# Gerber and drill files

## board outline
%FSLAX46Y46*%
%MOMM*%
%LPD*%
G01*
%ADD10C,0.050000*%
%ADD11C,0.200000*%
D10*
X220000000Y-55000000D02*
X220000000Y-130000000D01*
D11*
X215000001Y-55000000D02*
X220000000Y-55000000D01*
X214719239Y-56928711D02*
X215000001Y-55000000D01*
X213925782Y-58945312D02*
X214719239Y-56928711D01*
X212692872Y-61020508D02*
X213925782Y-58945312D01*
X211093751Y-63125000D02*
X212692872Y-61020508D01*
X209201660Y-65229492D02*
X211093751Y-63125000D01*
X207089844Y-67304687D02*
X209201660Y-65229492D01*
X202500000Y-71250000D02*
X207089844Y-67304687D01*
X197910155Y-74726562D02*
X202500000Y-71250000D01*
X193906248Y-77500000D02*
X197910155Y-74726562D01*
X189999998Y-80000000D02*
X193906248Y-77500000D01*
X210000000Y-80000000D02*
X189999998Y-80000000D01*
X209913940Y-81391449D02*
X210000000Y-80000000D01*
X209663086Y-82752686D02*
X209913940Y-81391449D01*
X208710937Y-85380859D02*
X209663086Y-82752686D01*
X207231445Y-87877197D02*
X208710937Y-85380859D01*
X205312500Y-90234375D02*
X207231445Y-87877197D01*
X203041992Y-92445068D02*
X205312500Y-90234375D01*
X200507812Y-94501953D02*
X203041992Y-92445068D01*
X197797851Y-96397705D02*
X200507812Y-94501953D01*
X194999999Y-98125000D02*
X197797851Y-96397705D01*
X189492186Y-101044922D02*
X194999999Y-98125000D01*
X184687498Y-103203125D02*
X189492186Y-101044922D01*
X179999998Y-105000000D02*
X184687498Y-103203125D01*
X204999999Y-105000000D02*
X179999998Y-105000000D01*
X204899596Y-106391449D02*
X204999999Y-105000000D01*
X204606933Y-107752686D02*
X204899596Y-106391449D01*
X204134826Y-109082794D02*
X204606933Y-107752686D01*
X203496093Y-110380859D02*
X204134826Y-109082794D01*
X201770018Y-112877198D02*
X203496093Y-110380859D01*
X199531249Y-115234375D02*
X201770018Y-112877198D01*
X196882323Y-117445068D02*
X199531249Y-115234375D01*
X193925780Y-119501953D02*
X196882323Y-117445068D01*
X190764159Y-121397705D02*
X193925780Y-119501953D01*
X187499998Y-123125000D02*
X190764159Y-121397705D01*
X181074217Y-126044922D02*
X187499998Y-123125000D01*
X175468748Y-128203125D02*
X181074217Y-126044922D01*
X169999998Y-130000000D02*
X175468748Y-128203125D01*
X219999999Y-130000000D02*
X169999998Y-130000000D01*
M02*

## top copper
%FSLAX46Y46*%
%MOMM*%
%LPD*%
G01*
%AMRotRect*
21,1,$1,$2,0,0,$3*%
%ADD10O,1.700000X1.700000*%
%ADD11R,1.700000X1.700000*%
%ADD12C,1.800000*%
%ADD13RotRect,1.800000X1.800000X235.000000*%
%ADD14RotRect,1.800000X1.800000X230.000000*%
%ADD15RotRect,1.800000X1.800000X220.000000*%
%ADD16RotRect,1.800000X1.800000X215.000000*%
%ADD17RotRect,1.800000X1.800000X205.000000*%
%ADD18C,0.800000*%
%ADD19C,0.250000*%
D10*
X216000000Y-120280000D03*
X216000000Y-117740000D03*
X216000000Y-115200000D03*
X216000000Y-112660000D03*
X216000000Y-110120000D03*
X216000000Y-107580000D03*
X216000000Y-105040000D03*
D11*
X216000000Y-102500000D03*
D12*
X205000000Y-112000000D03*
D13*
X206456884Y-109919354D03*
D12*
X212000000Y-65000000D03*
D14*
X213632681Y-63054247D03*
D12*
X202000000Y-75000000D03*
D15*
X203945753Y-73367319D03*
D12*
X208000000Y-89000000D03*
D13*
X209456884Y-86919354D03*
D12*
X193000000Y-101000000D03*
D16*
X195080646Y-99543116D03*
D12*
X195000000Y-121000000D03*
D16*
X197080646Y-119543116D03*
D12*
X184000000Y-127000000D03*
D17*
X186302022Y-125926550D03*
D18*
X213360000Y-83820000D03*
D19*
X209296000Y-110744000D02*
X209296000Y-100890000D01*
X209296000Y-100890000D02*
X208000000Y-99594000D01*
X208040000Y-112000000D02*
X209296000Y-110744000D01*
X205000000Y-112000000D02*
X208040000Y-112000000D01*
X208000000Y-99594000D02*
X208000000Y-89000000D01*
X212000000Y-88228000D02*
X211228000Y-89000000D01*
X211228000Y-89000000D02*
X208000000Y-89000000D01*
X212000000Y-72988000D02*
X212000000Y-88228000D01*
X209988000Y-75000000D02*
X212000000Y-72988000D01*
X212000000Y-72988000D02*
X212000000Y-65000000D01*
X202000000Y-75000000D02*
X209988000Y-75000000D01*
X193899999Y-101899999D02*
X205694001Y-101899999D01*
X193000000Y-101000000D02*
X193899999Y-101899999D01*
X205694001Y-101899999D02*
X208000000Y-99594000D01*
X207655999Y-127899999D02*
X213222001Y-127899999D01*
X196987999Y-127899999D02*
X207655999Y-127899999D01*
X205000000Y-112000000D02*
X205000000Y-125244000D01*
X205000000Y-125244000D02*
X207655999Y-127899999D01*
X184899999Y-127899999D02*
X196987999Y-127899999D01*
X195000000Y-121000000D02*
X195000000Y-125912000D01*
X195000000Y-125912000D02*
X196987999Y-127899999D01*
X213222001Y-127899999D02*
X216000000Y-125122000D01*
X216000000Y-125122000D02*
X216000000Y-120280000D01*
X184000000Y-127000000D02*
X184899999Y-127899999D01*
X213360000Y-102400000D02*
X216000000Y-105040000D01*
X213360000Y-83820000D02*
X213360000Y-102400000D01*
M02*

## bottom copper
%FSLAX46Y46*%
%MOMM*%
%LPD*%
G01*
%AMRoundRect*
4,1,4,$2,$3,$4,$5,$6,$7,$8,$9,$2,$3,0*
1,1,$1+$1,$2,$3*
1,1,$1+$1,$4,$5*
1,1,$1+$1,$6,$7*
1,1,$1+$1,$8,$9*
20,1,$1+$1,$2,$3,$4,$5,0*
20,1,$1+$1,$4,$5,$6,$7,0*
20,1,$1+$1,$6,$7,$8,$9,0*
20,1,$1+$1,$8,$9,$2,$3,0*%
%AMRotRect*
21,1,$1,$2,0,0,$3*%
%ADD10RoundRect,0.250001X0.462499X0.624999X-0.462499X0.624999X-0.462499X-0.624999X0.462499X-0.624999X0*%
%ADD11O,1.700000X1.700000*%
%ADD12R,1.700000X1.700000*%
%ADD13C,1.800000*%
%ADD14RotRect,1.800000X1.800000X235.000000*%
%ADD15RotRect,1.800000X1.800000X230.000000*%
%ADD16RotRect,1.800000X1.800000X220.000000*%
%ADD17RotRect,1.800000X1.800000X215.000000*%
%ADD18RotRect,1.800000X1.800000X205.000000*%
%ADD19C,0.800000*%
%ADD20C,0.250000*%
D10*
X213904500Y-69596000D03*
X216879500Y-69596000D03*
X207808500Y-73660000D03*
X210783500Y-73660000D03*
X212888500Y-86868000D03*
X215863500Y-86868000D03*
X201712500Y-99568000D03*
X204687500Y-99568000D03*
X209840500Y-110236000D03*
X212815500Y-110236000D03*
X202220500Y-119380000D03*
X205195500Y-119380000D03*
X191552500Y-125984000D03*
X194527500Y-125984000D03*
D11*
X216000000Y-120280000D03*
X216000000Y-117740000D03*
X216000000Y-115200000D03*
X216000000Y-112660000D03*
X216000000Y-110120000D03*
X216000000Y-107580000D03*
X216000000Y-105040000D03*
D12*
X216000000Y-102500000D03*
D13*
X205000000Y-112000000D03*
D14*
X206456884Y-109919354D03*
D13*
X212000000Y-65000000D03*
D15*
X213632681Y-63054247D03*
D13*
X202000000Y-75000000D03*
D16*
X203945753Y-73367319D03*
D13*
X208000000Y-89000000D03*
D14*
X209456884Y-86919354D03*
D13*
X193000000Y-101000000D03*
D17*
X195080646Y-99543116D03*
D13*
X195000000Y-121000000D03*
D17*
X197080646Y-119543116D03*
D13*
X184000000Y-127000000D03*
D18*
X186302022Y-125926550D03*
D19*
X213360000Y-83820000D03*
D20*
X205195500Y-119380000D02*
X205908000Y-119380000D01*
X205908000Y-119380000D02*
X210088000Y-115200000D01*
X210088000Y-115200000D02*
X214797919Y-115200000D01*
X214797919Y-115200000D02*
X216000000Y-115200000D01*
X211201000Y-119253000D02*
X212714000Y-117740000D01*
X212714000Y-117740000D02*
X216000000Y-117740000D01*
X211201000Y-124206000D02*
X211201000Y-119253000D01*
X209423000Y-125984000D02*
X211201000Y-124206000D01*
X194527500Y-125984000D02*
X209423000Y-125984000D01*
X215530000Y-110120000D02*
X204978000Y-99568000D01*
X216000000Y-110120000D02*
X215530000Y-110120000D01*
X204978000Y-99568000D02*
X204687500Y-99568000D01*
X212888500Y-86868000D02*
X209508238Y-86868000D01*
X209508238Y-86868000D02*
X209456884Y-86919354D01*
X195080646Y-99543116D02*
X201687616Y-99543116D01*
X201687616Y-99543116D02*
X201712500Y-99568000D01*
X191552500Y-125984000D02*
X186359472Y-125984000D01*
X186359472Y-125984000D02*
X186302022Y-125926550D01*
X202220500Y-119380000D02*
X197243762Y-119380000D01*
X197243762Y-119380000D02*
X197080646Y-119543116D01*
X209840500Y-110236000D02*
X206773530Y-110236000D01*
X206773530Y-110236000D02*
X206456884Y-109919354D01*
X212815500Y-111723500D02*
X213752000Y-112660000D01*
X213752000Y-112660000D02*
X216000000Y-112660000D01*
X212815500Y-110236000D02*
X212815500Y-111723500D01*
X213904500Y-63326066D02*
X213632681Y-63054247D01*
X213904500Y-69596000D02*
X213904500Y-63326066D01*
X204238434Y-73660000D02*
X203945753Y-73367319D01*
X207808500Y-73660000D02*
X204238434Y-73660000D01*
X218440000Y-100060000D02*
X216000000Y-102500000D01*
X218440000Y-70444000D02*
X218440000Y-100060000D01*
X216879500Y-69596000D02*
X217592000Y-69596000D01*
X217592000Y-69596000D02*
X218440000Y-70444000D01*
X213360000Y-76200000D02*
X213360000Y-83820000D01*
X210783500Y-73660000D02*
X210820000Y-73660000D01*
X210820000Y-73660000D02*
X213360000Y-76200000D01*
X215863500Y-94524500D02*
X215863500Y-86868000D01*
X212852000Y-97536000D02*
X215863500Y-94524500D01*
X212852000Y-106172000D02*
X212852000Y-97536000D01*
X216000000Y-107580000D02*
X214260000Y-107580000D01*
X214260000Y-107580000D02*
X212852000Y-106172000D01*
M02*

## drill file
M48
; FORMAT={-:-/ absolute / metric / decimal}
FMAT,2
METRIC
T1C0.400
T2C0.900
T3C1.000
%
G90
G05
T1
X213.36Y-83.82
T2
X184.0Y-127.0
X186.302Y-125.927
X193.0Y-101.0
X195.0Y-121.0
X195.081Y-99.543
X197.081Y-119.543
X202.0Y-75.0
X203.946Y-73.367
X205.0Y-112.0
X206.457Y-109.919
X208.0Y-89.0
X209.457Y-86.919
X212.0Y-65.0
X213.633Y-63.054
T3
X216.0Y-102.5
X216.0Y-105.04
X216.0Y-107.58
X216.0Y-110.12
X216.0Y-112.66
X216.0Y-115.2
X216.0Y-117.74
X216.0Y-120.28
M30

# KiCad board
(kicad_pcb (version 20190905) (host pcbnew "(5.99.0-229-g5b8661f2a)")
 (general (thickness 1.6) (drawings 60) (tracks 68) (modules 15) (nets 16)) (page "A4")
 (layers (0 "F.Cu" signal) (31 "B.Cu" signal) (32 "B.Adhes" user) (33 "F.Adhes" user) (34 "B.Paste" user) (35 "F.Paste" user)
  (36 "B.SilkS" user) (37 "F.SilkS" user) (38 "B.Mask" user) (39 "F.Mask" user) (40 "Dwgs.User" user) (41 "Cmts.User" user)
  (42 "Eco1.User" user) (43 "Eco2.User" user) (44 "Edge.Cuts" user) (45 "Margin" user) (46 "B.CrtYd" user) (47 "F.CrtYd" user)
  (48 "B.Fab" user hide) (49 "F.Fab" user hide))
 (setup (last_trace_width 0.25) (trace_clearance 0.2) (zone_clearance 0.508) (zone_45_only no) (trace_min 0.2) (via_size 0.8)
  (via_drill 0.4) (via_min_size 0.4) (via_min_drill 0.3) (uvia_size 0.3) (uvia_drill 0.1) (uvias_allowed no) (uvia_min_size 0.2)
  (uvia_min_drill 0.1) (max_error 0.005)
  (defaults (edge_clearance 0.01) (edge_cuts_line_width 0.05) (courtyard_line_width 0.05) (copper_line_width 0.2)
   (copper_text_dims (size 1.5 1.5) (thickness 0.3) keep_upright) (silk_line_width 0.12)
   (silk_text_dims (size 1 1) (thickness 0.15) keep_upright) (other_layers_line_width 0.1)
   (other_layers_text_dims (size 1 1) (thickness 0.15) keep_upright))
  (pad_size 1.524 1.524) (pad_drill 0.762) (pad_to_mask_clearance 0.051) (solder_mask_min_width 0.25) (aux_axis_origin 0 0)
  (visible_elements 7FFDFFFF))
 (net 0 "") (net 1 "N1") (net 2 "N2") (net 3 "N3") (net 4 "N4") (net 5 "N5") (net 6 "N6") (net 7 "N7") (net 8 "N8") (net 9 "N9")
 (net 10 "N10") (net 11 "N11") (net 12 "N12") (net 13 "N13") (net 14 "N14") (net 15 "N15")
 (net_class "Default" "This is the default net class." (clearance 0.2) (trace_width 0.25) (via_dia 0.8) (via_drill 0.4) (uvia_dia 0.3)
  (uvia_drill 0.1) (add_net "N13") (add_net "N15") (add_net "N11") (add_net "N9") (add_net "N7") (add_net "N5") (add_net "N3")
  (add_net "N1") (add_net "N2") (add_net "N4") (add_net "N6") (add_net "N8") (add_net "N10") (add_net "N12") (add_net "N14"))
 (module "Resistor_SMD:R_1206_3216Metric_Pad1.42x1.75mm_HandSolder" (layer "B.Cu") (at 215.392 69.596 180)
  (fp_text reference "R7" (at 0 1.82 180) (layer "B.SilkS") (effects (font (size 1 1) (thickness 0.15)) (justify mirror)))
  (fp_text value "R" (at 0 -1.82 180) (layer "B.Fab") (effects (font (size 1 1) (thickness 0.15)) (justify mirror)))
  (pad "2" smd roundrect (at 1.4875 0 180) (size 1.425 1.75) (layers "B.Cu" "B.Paste" "B.Mask") (roundrect_rratio 0.175439) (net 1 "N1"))
  (pad "1" smd roundrect (at -1.4875 0 180) (size 1.425 1.75) (layers "B.Cu" "B.Paste" "B.Mask") (roundrect_rratio 0.175439) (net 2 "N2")))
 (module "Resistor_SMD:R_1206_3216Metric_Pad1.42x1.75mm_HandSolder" (layer "B.Cu") (at 209.296 73.66 180)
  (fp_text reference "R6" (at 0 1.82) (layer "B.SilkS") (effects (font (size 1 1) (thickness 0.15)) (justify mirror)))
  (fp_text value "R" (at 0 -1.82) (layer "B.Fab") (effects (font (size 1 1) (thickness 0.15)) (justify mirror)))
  (pad "2" smd roundrect (at 1.4875 0 180) (size 1.425 1.75) (layers "B.Cu" "B.Paste" "B.Mask") (roundrect_rratio 0.175439) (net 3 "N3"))
  (pad "1" smd roundrect (at -1.4875 0 180) (size 1.425 1.75) (layers "B.Cu" "B.Paste" "B.Mask") (roundrect_rratio 0.175439) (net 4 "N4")))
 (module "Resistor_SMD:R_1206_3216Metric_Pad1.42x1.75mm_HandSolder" (layer "B.Cu") (at 214.376 86.868 180)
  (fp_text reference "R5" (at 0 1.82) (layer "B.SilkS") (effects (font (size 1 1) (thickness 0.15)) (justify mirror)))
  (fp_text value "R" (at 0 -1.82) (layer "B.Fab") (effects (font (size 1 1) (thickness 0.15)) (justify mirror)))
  (pad "2" smd roundrect (at 1.4875 0 180) (size 1.425 1.75) (layers "B.Cu" "B.Paste" "B.Mask") (roundrect_rratio 0.175439) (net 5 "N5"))
  (pad "1" smd roundrect (at -1.4875 0 180) (size 1.425 1.75) (layers "B.Cu" "B.Paste" "B.Mask") (roundrect_rratio 0.175439) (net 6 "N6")))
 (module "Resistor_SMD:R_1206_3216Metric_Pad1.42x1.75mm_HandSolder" (layer "B.Cu") (at 203.2 99.568 180)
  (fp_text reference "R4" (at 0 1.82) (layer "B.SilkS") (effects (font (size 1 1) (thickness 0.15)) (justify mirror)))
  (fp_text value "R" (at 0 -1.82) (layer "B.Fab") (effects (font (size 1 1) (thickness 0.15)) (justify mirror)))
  (pad "2" smd roundrect (at 1.4875 0 180) (size 1.425 1.75) (layers "B.Cu" "B.Paste" "B.Mask") (roundrect_rratio 0.175439) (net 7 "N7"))
  (pad "1" smd roundrect (at -1.4875 0 180) (size 1.425 1.75) (layers "B.Cu" "B.Paste" "B.Mask") (roundrect_rratio 0.175439) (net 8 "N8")))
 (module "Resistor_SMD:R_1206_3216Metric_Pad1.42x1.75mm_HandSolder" (layer "B.Cu") (at 211.328 110.236 180)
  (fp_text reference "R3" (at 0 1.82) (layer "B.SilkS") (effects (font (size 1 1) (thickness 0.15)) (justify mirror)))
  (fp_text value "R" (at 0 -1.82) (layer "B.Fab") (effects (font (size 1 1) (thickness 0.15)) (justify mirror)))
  (pad "2" smd roundrect (at 1.4875 0 180) (size 1.425 1.75) (layers "B.Cu" "B.Paste" "B.Mask") (roundrect_rratio 0.175439) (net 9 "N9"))
  (pad "1" smd roundrect (at -1.4875 0 180) (size 1.425 1.75) (layers "B.Cu" "B.Paste" "B.Mask") (roundrect_rratio 0.175439) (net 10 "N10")))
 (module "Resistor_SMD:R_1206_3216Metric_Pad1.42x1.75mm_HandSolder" (layer "B.Cu") (at 203.708 119.38 180)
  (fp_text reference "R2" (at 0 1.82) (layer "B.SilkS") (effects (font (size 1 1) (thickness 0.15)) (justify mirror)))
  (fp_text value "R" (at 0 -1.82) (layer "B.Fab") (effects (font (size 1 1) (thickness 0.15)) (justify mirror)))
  (pad "2" smd roundrect (at 1.4875 0 180) (size 1.425 1.75) (layers "B.Cu" "B.Paste" "B.Mask") (roundrect_rratio 0.175439) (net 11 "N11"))
  (pad "1" smd roundrect (at -1.4875 0 180) (size 1.425 1.75) (layers "B.Cu" "B.Paste" "B.Mask") (roundrect_rratio 0.175439) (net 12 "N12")))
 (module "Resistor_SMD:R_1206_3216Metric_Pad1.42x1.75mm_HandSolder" (layer "B.Cu") (at 193.04 125.984 180)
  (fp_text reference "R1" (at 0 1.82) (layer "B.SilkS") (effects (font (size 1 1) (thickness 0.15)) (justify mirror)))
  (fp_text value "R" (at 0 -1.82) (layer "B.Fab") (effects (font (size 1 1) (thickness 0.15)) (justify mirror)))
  (pad "2" smd roundrect (at 1.4875 0 180) (size 1.425 1.75) (layers "B.Cu" "B.Paste" "B.Mask") (roundrect_rratio 0.175439) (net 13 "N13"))
  (pad "1" smd roundrect (at -1.4875 0 180) (size 1.425 1.75) (layers "B.Cu" "B.Paste" "B.Mask") (roundrect_rratio 0.175439) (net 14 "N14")))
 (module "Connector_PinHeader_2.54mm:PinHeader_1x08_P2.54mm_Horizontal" (layer "F.Cu") (at 216 102.5)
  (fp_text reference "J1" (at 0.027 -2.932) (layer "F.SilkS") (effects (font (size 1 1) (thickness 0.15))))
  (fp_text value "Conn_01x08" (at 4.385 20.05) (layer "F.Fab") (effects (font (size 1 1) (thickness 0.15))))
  (pad "8" thru_hole oval (at 0 17.78) (size 1.7 1.7) (drill 1) (layers *.Cu *.Mask) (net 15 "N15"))
  (pad "7" thru_hole oval (at 0 15.24) (size 1.7 1.7) (drill 1) (layers *.Cu *.Mask) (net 14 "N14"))
  (pad "6" thru_hole oval (at 0 12.7) (size 1.7 1.7) (drill 1) (layers *.Cu *.Mask) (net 12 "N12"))
  (pad "5" thru_hole oval (at 0 10.16) (size 1.7 1.7) (drill 1) (layers *.Cu *.Mask) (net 10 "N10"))
  (pad "4" thru_hole oval (at 0 7.62) (size 1.7 1.7) (drill 1) (layers *.Cu *.Mask) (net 8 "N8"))
  (pad "3" thru_hole oval (at 0 5.08) (size 1.7 1.7) (drill 1) (layers *.Cu *.Mask) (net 6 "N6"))
  (pad "2" thru_hole oval (at 0 2.54) (size 1.7 1.7) (drill 1) (layers *.Cu *.Mask) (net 4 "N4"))
  (pad "1" thru_hole rect (at 0 0) (size 1.7 1.7) (drill 1) (layers *.Cu *.Mask) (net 2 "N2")))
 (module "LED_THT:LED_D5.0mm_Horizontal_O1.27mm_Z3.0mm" (layer "F.Cu") (at 206.456884 109.919354 -125)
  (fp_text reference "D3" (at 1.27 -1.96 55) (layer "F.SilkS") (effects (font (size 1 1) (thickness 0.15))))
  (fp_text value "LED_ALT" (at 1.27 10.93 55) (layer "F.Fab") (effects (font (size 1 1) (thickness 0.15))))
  (pad "2" thru_hole circle (at 2.54 0 235) (size 1.8 1.8) (drill 0.9) (layers *.Cu *.Mask) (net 15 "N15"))
  (pad "1" thru_hole rect (at 0 0 235) (size 1.8 1.8) (drill 0.9) (layers *.Cu *.Mask) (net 9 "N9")))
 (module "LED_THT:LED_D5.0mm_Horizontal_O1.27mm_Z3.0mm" (layer "F.Cu") (at 213.632681 63.054247 -130)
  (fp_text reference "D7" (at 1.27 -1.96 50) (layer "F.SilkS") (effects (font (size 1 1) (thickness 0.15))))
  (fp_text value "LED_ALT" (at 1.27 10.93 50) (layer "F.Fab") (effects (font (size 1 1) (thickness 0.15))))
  (pad "2" thru_hole circle (at 2.54 0 230) (size 1.8 1.8) (drill 0.9) (layers *.Cu *.Mask) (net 15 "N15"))
  (pad "1" thru_hole rect (at 0 0 230) (size 1.8 1.8) (drill 0.9) (layers *.Cu *.Mask) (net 1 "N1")))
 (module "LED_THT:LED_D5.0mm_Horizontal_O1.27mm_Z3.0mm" (layer "F.Cu") (at 203.945753 73.367319 -140)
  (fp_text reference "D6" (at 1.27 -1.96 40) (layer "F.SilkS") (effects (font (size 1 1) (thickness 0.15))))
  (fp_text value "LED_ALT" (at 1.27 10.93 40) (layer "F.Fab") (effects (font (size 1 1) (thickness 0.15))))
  (pad "2" thru_hole circle (at 2.54 0 220) (size 1.8 1.8) (drill 0.9) (layers *.Cu *.Mask) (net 15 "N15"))
  (pad "1" thru_hole rect (at 0 0 220) (size 1.8 1.8) (drill 0.9) (layers *.Cu *.Mask) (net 3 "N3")))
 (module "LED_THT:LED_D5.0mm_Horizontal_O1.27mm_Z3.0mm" (layer "F.Cu") (at 209.456884 86.919354 -125)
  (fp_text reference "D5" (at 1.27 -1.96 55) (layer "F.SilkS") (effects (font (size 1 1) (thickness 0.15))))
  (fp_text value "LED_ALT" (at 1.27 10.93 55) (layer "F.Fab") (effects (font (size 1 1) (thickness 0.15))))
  (pad "2" thru_hole circle (at 2.54 0 235) (size 1.8 1.8) (drill 0.9) (layers *.Cu *.Mask) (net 15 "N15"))
  (pad "1" thru_hole rect (at 0 0 235) (size 1.8 1.8) (drill 0.9) (layers *.Cu *.Mask) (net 5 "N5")))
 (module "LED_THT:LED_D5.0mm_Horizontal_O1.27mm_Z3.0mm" (layer "F.Cu") (at 195.080646 99.543116 -145)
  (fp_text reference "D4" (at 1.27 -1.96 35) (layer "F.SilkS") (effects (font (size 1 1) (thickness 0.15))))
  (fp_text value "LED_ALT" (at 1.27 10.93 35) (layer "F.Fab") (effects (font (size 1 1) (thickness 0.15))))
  (pad "2" thru_hole circle (at 2.54 0 215) (size 1.8 1.8) (drill 0.9) (layers *.Cu *.Mask) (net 15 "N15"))
  (pad "1" thru_hole rect (at 0 0 215) (size 1.8 1.8) (drill 0.9) (layers *.Cu *.Mask) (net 7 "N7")))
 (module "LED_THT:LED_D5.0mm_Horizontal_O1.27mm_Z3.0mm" (layer "F.Cu") (at 197.080646 119.543116 -145)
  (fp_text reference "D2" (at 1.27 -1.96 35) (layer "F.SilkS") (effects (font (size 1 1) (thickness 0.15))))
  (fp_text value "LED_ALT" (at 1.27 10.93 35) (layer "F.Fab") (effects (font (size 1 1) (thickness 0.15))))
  (pad "2" thru_hole circle (at 2.54 0 215) (size 1.8 1.8) (drill 0.9) (layers *.Cu *.Mask) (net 15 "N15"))
  (pad "1" thru_hole rect (at 0 0 215) (size 1.8 1.8) (drill 0.9) (layers *.Cu *.Mask) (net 11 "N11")))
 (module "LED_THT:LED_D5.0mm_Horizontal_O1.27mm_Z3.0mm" (layer "F.Cu") (at 186.302022 125.92655 -155)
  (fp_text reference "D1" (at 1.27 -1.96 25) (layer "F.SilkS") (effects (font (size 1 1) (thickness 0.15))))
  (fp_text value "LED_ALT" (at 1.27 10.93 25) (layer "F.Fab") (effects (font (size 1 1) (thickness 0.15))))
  (pad "2" thru_hole circle (at 2.54 0 205) (size 1.8 1.8) (drill 0.9) (layers *.Cu *.Mask) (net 15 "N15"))
  (pad "1" thru_hole rect (at 0 0 205) (size 1.8 1.8) (drill 0.9) (layers *.Cu *.Mask) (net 13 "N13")))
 (gr_line (start 220 55) (end 220 130) (layer "Edge.Cuts") (width 0.05))
 (gr_line (start 215.000001 55) (end 220 55) (layer "Edge.Cuts") (width 0.2))
 (gr_line (start 214.719239 56.928711) (end 215.000001 55) (layer "Edge.Cuts") (width 0.2))
 (gr_line (start 213.925782 58.945312) (end 214.719239 56.928711) (layer "Edge.Cuts") (width 0.2))
 (gr_line (start 212.692872 61.020508) (end 213.925782 58.945312) (layer "Edge.Cuts") (width 0.2))
 (gr_line (start 211.093751 63.125) (end 212.692872 61.020508) (layer "Edge.Cuts") (width 0.2))
 (gr_line (start 209.20166 65.229492) (end 211.093751 63.125) (layer "Edge.Cuts") (width 0.2))
 (gr_line (start 207.089844 67.304687) (end 209.20166 65.229492) (layer "Edge.Cuts") (width 0.2))
 (gr_line (start 202.5 71.25) (end 207.089844 67.304687) (layer "Edge.Cuts") (width 0.2))
 (gr_line (start 197.910155 74.726562) (end 202.5 71.25) (layer "Edge.Cuts") (width 0.2))
 (gr_line (start 193.906248 77.5) (end 197.910155 74.726562) (layer "Edge.Cuts") (width 0.2))
 (gr_line (start 189.999998 80) (end 193.906248 77.5) (layer "Edge.Cuts") (width 0.2))
 (gr_line (start 210 80) (end 189.999998 80) (layer "Edge.Cuts") (width 0.2))
 (gr_line (start 209.91394 81.391449) (end 210 80) (layer "Edge.Cuts") (width 0.2))
 (gr_line (start 209.663086 82.752686) (end 209.91394 81.391449) (layer "Edge.Cuts") (width 0.2))
 (gr_line (start 208.710937 85.380859) (end 209.663086 82.752686) (layer "Edge.Cuts") (width 0.2))
 (gr_line (start 207.231445 87.877197) (end 208.710937 85.380859) (layer "Edge.Cuts") (width 0.2))
 (gr_line (start 205.3125 90.234375) (end 207.231445 87.877197) (layer "Edge.Cuts") (width 0.2))
 (gr_line (start 203.041992 92.445068) (end 205.3125 90.234375) (layer "Edge.Cuts") (width 0.2))
 (gr_line (start 200.507812 94.501953) (end 203.041992 92.445068) (layer "Edge.Cuts") (width 0.2))
 (gr_line (start 197.797851 96.397705) (end 200.507812 94.501953) (layer "Edge.Cuts") (width 0.2))
 (gr_line (start 194.999999 98.125) (end 197.797851 96.397705) (layer "Edge.Cuts") (width 0.2))
 (gr_line (start 189.492186 101.044922) (end 194.999999 98.125) (layer "Edge.Cuts") (width 0.2))
 (gr_line (start 184.687498 103.203125) (end 189.492186 101.044922) (layer "Edge.Cuts") (width 0.2))
 (gr_line (start 179.999998 105) (end 184.687498 103.203125) (layer "Edge.Cuts") (width 0.2))
 (gr_line (start 204.999999 105) (end 179.999998 105) (layer "Edge.Cuts") (width 0.2))
 (gr_line (start 204.899596 106.391449) (end 204.999999 105) (layer "Edge.Cuts") (width 0.2))
 (gr_line (start 204.606933 107.752686) (end 204.899596 106.391449) (layer "Edge.Cuts") (width 0.2))
 (gr_line (start 204.134826 109.082794) (end 204.606933 107.752686) (layer "Edge.Cuts") (width 0.2))
 (gr_line (start 203.496093 110.380859) (end 204.134826 109.082794) (layer "Edge.Cuts") (width 0.2))
 (gr_line (start 201.770018 112.877198) (end 203.496093 110.380859) (layer "Edge.Cuts") (width 0.2))
 (gr_line (start 199.531249 115.234375) (end 201.770018 112.877198) (layer "Edge.Cuts") (width 0.2))
 (gr_line (start 196.882323 117.445068) (end 199.531249 115.234375) (layer "Edge.Cuts") (width 0.2))
 (gr_line (start 193.92578 119.501953) (end 196.882323 117.445068) (layer "Edge.Cuts") (width 0.2))
 (gr_line (start 190.764159 121.397705) (end 193.92578 119.501953) (layer "Edge.Cuts") (width 0.2))
 (gr_line (start 187.499998 123.125) (end 190.764159 121.397705) (layer "Edge.Cuts") (width 0.2))
 (gr_line (start 181.074217 126.044922) (end 187.499998 123.125) (layer "Edge.Cuts") (width 0.2))
 (gr_line (start 175.468748 128.203125) (end 181.074217 126.044922) (layer "Edge.Cuts") (width 0.2))
 (gr_line (start 169.999998 130) (end 175.468748 128.203125) (layer "Edge.Cuts") (width 0.2))
 (gr_line (start 219.999999 130) (end 169.999998 130) (layer "Edge.Cuts") (width 0.2))
 (segment (start 205.1955 119.38) (end 205.908 119.38) (width 0.25) (layer "B.Cu") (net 12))
 (segment (start 205.908 119.38) (end 210.088 115.2) (width 0.25) (layer "B.Cu") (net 12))
 (segment (start 210.088 115.2) (end 214.797919 115.2) (width 0.25) (layer "B.Cu") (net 12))
 (segment (start 214.797919 115.2) (end 216 115.2) (width 0.25) (layer "B.Cu") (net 12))
 (segment (start 211.201 119.253) (end 212.714 117.74) (width 0.25) (layer "B.Cu") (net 14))
 (segment (start 212.714 117.74) (end 216 117.74) (width 0.25) (layer "B.Cu") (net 14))
 (segment (start 211.201 124.206) (end 211.201 119.253) (width 0.25) (layer "B.Cu") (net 14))
 (segment (start 209.423 125.984) (end 211.201 124.206) (width 0.25) (layer "B.Cu") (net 14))
 (segment (start 194.5275 125.984) (end 209.423 125.984) (width 0.25) (layer "B.Cu") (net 14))
 (segment (start 215.53 110.12) (end 204.978 99.568) (width 0.25) (layer "B.Cu") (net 8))
 (segment (start 216 110.12) (end 215.53 110.12) (width 0.25) (layer "B.Cu") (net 8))
 (segment (start 204.978 99.568) (end 204.6875 99.568) (width 0.25) (layer "B.Cu") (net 8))
 (segment (start 212.8885 86.868) (end 209.508238 86.868) (width 0.25) (layer "B.Cu") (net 5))
 (segment (start 209.508238 86.868) (end 209.456884 86.919354) (width 0.25) (layer "B.Cu") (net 5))
 (segment (start 195.080646 99.543116) (end 201.687616 99.543116) (width 0.25) (layer "B.Cu") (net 7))
 (segment (start 201.687616 99.543116) (end 201.7125 99.568) (width 0.25) (layer "B.Cu") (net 7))
 (segment (start 191.5525 125.984) (end 186.359472 125.984) (width 0.25) (layer "B.Cu") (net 13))
 (segment (start 186.359472 125.984) (end 186.302022 125.92655) (width 0.25) (layer "B.Cu") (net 13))
 (segment (start 202.2205 119.38) (end 197.243762 119.38) (width 0.25) (layer "B.Cu") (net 11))
 (segment (start 197.243762 119.38) (end 197.080646 119.543116) (width 0.25) (layer "B.Cu") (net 11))
 (segment (start 209.8405 110.236) (end 206.77353 110.236) (width 0.25) (layer "B.Cu") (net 9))
 (segment (start 206.77353 110.236) (end 206.456884 109.919354) (width 0.25) (layer "B.Cu") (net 9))
 (segment (start 212.8155 111.7235) (end 213.752 112.66) (width 0.25) (layer "B.Cu") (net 10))
 (segment (start 213.752 112.66) (end 216 112.66) (width 0.25) (layer "B.Cu") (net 10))
 (segment (start 212.8155 110.236) (end 212.8155 111.7235) (width 0.25) (layer "B.Cu") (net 10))
 (segment (start 209.296 110.744) (end 209.296 100.89) (width 0.25) (layer "F.Cu") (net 15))
 (segment (start 209.296 100.89) (end 208 99.594) (width 0.25) (layer "F.Cu") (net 15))
 (segment (start 208.04 112) (end 209.296 110.744) (width 0.25) (layer "F.Cu") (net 15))
 (segment (start 205 112) (end 208.04 112) (width 0.25) (layer "F.Cu") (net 15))
 (segment (start 208 99.594) (end 208 89) (width 0.25) (layer "F.Cu") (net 15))
 (segment (start 212 88.228) (end 211.228 89) (width 0.25) (layer "F.Cu") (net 15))
 (segment (start 211.228 89) (end 208 89) (width 0.25) (layer "F.Cu") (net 15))
 (segment (start 212 72.988) (end 212 88.228) (width 0.25) (layer "F.Cu") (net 15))
 (segment (start 209.988 75) (end 212 72.988) (width 0.25) (layer "F.Cu") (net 15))
 (segment (start 212 72.988) (end 212 65) (width 0.25) (layer "F.Cu") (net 15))
 (segment (start 202 75) (end 209.988 75) (width 0.25) (layer "F.Cu") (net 15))
 (segment (start 193.899999 101.899999) (end 205.694001 101.899999) (width 0.25) (layer "F.Cu") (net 15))
 (segment (start 193 101) (end 193.899999 101.899999) (width 0.25) (layer "F.Cu") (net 15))
 (segment (start 205.694001 101.899999) (end 208 99.594) (width 0.25) (layer "F.Cu") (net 15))
 (segment (start 207.655999 127.899999) (end 213.222001 127.899999) (width 0.25) (layer "F.Cu") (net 15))
 (segment (start 196.987999 127.899999) (end 207.655999 127.899999) (width 0.25) (layer "F.Cu") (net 15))
 (segment (start 205 112) (end 205 125.244) (width 0.25) (layer "F.Cu") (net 15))
 (segment (start 205 125.244) (end 207.655999 127.899999) (width 0.25) (layer "F.Cu") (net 15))
 (segment (start 184.899999 127.899999) (end 196.987999 127.899999) (width 0.25) (layer "F.Cu") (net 15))
 (segment (start 195 121) (end 195 125.912) (width 0.25) (layer "F.Cu") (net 15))
 (segment (start 195 125.912) (end 196.987999 127.899999) (width 0.25) (layer "F.Cu") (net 15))
 (segment (start 213.222001 127.899999) (end 216 125.122) (width 0.25) (layer "F.Cu") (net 15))
 (segment (start 216 125.122) (end 216 120.28) (width 0.25) (layer "F.Cu") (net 15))
 (segment (start 184 127) (end 184.899999 127.899999) (width 0.25) (layer "F.Cu") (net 15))
 (segment (start 213.9045 63.326066) (end 213.632681 63.054247) (width 0.25) (layer "B.Cu") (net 1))
 (segment (start 213.9045 69.596) (end 213.9045 63.326066) (width 0.25) (layer "B.Cu") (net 1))
 (segment (start 204.238434 73.66) (end 203.945753 73.367319) (width 0.25) (layer "B.Cu") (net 3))
 (segment (start 207.8085 73.66) (end 204.238434 73.66) (width 0.25) (layer "B.Cu") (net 3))
 (segment (start 218.44 100.06) (end 216 102.5) (width 0.25) (layer "B.Cu") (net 2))
 (segment (start 218.44 70.444) (end 218.44 100.06) (width 0.25) (layer "B.Cu") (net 2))
 (segment (start 216.8795 69.596) (end 217.592 69.596) (width 0.25) (layer "B.Cu") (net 2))
 (segment (start 217.592 69.596) (end 218.44 70.444) (width 0.25) (layer "B.Cu") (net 2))
 (via (at 213.36 83.82) (size 0.8) (drill 0.4) (layers "F.Cu" "B.Cu") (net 4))
 (segment (start 213.36 76.2) (end 213.36 83.82) (width 0.25) (layer "B.Cu") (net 4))
 (segment (start 210.7835 73.66) (end 210.82 73.66) (width 0.25) (layer "B.Cu") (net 4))
 (segment (start 210.82 73.66) (end 213.36 76.2) (width 0.25) (layer "B.Cu") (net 4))
 (segment (start 213.36 102.4) (end 216 105.04) (width 0.25) (layer "F.Cu") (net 4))
 (segment (start 213.36 83.82) (end 213.36 102.4) (width 0.25) (layer "F.Cu") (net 4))
 (segment (start 215.8635 94.5245) (end 215.8635 86.868) (width 0.25) (layer "B.Cu") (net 6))
 (segment (start 212.852 97.536) (end 215.8635 94.5245) (width 0.25) (layer "B.Cu") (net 6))
 (segment (start 212.852 106.172) (end 212.852 97.536) (width 0.25) (layer "B.Cu") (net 6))
 (segment (start 216 107.58) (end 214.26 107.58) (width 0.25) (layer "B.Cu") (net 6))
 (segment (start 214.26 107.58) (end 212.852 106.172) (width 0.25) (layer "B.Cu") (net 6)))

